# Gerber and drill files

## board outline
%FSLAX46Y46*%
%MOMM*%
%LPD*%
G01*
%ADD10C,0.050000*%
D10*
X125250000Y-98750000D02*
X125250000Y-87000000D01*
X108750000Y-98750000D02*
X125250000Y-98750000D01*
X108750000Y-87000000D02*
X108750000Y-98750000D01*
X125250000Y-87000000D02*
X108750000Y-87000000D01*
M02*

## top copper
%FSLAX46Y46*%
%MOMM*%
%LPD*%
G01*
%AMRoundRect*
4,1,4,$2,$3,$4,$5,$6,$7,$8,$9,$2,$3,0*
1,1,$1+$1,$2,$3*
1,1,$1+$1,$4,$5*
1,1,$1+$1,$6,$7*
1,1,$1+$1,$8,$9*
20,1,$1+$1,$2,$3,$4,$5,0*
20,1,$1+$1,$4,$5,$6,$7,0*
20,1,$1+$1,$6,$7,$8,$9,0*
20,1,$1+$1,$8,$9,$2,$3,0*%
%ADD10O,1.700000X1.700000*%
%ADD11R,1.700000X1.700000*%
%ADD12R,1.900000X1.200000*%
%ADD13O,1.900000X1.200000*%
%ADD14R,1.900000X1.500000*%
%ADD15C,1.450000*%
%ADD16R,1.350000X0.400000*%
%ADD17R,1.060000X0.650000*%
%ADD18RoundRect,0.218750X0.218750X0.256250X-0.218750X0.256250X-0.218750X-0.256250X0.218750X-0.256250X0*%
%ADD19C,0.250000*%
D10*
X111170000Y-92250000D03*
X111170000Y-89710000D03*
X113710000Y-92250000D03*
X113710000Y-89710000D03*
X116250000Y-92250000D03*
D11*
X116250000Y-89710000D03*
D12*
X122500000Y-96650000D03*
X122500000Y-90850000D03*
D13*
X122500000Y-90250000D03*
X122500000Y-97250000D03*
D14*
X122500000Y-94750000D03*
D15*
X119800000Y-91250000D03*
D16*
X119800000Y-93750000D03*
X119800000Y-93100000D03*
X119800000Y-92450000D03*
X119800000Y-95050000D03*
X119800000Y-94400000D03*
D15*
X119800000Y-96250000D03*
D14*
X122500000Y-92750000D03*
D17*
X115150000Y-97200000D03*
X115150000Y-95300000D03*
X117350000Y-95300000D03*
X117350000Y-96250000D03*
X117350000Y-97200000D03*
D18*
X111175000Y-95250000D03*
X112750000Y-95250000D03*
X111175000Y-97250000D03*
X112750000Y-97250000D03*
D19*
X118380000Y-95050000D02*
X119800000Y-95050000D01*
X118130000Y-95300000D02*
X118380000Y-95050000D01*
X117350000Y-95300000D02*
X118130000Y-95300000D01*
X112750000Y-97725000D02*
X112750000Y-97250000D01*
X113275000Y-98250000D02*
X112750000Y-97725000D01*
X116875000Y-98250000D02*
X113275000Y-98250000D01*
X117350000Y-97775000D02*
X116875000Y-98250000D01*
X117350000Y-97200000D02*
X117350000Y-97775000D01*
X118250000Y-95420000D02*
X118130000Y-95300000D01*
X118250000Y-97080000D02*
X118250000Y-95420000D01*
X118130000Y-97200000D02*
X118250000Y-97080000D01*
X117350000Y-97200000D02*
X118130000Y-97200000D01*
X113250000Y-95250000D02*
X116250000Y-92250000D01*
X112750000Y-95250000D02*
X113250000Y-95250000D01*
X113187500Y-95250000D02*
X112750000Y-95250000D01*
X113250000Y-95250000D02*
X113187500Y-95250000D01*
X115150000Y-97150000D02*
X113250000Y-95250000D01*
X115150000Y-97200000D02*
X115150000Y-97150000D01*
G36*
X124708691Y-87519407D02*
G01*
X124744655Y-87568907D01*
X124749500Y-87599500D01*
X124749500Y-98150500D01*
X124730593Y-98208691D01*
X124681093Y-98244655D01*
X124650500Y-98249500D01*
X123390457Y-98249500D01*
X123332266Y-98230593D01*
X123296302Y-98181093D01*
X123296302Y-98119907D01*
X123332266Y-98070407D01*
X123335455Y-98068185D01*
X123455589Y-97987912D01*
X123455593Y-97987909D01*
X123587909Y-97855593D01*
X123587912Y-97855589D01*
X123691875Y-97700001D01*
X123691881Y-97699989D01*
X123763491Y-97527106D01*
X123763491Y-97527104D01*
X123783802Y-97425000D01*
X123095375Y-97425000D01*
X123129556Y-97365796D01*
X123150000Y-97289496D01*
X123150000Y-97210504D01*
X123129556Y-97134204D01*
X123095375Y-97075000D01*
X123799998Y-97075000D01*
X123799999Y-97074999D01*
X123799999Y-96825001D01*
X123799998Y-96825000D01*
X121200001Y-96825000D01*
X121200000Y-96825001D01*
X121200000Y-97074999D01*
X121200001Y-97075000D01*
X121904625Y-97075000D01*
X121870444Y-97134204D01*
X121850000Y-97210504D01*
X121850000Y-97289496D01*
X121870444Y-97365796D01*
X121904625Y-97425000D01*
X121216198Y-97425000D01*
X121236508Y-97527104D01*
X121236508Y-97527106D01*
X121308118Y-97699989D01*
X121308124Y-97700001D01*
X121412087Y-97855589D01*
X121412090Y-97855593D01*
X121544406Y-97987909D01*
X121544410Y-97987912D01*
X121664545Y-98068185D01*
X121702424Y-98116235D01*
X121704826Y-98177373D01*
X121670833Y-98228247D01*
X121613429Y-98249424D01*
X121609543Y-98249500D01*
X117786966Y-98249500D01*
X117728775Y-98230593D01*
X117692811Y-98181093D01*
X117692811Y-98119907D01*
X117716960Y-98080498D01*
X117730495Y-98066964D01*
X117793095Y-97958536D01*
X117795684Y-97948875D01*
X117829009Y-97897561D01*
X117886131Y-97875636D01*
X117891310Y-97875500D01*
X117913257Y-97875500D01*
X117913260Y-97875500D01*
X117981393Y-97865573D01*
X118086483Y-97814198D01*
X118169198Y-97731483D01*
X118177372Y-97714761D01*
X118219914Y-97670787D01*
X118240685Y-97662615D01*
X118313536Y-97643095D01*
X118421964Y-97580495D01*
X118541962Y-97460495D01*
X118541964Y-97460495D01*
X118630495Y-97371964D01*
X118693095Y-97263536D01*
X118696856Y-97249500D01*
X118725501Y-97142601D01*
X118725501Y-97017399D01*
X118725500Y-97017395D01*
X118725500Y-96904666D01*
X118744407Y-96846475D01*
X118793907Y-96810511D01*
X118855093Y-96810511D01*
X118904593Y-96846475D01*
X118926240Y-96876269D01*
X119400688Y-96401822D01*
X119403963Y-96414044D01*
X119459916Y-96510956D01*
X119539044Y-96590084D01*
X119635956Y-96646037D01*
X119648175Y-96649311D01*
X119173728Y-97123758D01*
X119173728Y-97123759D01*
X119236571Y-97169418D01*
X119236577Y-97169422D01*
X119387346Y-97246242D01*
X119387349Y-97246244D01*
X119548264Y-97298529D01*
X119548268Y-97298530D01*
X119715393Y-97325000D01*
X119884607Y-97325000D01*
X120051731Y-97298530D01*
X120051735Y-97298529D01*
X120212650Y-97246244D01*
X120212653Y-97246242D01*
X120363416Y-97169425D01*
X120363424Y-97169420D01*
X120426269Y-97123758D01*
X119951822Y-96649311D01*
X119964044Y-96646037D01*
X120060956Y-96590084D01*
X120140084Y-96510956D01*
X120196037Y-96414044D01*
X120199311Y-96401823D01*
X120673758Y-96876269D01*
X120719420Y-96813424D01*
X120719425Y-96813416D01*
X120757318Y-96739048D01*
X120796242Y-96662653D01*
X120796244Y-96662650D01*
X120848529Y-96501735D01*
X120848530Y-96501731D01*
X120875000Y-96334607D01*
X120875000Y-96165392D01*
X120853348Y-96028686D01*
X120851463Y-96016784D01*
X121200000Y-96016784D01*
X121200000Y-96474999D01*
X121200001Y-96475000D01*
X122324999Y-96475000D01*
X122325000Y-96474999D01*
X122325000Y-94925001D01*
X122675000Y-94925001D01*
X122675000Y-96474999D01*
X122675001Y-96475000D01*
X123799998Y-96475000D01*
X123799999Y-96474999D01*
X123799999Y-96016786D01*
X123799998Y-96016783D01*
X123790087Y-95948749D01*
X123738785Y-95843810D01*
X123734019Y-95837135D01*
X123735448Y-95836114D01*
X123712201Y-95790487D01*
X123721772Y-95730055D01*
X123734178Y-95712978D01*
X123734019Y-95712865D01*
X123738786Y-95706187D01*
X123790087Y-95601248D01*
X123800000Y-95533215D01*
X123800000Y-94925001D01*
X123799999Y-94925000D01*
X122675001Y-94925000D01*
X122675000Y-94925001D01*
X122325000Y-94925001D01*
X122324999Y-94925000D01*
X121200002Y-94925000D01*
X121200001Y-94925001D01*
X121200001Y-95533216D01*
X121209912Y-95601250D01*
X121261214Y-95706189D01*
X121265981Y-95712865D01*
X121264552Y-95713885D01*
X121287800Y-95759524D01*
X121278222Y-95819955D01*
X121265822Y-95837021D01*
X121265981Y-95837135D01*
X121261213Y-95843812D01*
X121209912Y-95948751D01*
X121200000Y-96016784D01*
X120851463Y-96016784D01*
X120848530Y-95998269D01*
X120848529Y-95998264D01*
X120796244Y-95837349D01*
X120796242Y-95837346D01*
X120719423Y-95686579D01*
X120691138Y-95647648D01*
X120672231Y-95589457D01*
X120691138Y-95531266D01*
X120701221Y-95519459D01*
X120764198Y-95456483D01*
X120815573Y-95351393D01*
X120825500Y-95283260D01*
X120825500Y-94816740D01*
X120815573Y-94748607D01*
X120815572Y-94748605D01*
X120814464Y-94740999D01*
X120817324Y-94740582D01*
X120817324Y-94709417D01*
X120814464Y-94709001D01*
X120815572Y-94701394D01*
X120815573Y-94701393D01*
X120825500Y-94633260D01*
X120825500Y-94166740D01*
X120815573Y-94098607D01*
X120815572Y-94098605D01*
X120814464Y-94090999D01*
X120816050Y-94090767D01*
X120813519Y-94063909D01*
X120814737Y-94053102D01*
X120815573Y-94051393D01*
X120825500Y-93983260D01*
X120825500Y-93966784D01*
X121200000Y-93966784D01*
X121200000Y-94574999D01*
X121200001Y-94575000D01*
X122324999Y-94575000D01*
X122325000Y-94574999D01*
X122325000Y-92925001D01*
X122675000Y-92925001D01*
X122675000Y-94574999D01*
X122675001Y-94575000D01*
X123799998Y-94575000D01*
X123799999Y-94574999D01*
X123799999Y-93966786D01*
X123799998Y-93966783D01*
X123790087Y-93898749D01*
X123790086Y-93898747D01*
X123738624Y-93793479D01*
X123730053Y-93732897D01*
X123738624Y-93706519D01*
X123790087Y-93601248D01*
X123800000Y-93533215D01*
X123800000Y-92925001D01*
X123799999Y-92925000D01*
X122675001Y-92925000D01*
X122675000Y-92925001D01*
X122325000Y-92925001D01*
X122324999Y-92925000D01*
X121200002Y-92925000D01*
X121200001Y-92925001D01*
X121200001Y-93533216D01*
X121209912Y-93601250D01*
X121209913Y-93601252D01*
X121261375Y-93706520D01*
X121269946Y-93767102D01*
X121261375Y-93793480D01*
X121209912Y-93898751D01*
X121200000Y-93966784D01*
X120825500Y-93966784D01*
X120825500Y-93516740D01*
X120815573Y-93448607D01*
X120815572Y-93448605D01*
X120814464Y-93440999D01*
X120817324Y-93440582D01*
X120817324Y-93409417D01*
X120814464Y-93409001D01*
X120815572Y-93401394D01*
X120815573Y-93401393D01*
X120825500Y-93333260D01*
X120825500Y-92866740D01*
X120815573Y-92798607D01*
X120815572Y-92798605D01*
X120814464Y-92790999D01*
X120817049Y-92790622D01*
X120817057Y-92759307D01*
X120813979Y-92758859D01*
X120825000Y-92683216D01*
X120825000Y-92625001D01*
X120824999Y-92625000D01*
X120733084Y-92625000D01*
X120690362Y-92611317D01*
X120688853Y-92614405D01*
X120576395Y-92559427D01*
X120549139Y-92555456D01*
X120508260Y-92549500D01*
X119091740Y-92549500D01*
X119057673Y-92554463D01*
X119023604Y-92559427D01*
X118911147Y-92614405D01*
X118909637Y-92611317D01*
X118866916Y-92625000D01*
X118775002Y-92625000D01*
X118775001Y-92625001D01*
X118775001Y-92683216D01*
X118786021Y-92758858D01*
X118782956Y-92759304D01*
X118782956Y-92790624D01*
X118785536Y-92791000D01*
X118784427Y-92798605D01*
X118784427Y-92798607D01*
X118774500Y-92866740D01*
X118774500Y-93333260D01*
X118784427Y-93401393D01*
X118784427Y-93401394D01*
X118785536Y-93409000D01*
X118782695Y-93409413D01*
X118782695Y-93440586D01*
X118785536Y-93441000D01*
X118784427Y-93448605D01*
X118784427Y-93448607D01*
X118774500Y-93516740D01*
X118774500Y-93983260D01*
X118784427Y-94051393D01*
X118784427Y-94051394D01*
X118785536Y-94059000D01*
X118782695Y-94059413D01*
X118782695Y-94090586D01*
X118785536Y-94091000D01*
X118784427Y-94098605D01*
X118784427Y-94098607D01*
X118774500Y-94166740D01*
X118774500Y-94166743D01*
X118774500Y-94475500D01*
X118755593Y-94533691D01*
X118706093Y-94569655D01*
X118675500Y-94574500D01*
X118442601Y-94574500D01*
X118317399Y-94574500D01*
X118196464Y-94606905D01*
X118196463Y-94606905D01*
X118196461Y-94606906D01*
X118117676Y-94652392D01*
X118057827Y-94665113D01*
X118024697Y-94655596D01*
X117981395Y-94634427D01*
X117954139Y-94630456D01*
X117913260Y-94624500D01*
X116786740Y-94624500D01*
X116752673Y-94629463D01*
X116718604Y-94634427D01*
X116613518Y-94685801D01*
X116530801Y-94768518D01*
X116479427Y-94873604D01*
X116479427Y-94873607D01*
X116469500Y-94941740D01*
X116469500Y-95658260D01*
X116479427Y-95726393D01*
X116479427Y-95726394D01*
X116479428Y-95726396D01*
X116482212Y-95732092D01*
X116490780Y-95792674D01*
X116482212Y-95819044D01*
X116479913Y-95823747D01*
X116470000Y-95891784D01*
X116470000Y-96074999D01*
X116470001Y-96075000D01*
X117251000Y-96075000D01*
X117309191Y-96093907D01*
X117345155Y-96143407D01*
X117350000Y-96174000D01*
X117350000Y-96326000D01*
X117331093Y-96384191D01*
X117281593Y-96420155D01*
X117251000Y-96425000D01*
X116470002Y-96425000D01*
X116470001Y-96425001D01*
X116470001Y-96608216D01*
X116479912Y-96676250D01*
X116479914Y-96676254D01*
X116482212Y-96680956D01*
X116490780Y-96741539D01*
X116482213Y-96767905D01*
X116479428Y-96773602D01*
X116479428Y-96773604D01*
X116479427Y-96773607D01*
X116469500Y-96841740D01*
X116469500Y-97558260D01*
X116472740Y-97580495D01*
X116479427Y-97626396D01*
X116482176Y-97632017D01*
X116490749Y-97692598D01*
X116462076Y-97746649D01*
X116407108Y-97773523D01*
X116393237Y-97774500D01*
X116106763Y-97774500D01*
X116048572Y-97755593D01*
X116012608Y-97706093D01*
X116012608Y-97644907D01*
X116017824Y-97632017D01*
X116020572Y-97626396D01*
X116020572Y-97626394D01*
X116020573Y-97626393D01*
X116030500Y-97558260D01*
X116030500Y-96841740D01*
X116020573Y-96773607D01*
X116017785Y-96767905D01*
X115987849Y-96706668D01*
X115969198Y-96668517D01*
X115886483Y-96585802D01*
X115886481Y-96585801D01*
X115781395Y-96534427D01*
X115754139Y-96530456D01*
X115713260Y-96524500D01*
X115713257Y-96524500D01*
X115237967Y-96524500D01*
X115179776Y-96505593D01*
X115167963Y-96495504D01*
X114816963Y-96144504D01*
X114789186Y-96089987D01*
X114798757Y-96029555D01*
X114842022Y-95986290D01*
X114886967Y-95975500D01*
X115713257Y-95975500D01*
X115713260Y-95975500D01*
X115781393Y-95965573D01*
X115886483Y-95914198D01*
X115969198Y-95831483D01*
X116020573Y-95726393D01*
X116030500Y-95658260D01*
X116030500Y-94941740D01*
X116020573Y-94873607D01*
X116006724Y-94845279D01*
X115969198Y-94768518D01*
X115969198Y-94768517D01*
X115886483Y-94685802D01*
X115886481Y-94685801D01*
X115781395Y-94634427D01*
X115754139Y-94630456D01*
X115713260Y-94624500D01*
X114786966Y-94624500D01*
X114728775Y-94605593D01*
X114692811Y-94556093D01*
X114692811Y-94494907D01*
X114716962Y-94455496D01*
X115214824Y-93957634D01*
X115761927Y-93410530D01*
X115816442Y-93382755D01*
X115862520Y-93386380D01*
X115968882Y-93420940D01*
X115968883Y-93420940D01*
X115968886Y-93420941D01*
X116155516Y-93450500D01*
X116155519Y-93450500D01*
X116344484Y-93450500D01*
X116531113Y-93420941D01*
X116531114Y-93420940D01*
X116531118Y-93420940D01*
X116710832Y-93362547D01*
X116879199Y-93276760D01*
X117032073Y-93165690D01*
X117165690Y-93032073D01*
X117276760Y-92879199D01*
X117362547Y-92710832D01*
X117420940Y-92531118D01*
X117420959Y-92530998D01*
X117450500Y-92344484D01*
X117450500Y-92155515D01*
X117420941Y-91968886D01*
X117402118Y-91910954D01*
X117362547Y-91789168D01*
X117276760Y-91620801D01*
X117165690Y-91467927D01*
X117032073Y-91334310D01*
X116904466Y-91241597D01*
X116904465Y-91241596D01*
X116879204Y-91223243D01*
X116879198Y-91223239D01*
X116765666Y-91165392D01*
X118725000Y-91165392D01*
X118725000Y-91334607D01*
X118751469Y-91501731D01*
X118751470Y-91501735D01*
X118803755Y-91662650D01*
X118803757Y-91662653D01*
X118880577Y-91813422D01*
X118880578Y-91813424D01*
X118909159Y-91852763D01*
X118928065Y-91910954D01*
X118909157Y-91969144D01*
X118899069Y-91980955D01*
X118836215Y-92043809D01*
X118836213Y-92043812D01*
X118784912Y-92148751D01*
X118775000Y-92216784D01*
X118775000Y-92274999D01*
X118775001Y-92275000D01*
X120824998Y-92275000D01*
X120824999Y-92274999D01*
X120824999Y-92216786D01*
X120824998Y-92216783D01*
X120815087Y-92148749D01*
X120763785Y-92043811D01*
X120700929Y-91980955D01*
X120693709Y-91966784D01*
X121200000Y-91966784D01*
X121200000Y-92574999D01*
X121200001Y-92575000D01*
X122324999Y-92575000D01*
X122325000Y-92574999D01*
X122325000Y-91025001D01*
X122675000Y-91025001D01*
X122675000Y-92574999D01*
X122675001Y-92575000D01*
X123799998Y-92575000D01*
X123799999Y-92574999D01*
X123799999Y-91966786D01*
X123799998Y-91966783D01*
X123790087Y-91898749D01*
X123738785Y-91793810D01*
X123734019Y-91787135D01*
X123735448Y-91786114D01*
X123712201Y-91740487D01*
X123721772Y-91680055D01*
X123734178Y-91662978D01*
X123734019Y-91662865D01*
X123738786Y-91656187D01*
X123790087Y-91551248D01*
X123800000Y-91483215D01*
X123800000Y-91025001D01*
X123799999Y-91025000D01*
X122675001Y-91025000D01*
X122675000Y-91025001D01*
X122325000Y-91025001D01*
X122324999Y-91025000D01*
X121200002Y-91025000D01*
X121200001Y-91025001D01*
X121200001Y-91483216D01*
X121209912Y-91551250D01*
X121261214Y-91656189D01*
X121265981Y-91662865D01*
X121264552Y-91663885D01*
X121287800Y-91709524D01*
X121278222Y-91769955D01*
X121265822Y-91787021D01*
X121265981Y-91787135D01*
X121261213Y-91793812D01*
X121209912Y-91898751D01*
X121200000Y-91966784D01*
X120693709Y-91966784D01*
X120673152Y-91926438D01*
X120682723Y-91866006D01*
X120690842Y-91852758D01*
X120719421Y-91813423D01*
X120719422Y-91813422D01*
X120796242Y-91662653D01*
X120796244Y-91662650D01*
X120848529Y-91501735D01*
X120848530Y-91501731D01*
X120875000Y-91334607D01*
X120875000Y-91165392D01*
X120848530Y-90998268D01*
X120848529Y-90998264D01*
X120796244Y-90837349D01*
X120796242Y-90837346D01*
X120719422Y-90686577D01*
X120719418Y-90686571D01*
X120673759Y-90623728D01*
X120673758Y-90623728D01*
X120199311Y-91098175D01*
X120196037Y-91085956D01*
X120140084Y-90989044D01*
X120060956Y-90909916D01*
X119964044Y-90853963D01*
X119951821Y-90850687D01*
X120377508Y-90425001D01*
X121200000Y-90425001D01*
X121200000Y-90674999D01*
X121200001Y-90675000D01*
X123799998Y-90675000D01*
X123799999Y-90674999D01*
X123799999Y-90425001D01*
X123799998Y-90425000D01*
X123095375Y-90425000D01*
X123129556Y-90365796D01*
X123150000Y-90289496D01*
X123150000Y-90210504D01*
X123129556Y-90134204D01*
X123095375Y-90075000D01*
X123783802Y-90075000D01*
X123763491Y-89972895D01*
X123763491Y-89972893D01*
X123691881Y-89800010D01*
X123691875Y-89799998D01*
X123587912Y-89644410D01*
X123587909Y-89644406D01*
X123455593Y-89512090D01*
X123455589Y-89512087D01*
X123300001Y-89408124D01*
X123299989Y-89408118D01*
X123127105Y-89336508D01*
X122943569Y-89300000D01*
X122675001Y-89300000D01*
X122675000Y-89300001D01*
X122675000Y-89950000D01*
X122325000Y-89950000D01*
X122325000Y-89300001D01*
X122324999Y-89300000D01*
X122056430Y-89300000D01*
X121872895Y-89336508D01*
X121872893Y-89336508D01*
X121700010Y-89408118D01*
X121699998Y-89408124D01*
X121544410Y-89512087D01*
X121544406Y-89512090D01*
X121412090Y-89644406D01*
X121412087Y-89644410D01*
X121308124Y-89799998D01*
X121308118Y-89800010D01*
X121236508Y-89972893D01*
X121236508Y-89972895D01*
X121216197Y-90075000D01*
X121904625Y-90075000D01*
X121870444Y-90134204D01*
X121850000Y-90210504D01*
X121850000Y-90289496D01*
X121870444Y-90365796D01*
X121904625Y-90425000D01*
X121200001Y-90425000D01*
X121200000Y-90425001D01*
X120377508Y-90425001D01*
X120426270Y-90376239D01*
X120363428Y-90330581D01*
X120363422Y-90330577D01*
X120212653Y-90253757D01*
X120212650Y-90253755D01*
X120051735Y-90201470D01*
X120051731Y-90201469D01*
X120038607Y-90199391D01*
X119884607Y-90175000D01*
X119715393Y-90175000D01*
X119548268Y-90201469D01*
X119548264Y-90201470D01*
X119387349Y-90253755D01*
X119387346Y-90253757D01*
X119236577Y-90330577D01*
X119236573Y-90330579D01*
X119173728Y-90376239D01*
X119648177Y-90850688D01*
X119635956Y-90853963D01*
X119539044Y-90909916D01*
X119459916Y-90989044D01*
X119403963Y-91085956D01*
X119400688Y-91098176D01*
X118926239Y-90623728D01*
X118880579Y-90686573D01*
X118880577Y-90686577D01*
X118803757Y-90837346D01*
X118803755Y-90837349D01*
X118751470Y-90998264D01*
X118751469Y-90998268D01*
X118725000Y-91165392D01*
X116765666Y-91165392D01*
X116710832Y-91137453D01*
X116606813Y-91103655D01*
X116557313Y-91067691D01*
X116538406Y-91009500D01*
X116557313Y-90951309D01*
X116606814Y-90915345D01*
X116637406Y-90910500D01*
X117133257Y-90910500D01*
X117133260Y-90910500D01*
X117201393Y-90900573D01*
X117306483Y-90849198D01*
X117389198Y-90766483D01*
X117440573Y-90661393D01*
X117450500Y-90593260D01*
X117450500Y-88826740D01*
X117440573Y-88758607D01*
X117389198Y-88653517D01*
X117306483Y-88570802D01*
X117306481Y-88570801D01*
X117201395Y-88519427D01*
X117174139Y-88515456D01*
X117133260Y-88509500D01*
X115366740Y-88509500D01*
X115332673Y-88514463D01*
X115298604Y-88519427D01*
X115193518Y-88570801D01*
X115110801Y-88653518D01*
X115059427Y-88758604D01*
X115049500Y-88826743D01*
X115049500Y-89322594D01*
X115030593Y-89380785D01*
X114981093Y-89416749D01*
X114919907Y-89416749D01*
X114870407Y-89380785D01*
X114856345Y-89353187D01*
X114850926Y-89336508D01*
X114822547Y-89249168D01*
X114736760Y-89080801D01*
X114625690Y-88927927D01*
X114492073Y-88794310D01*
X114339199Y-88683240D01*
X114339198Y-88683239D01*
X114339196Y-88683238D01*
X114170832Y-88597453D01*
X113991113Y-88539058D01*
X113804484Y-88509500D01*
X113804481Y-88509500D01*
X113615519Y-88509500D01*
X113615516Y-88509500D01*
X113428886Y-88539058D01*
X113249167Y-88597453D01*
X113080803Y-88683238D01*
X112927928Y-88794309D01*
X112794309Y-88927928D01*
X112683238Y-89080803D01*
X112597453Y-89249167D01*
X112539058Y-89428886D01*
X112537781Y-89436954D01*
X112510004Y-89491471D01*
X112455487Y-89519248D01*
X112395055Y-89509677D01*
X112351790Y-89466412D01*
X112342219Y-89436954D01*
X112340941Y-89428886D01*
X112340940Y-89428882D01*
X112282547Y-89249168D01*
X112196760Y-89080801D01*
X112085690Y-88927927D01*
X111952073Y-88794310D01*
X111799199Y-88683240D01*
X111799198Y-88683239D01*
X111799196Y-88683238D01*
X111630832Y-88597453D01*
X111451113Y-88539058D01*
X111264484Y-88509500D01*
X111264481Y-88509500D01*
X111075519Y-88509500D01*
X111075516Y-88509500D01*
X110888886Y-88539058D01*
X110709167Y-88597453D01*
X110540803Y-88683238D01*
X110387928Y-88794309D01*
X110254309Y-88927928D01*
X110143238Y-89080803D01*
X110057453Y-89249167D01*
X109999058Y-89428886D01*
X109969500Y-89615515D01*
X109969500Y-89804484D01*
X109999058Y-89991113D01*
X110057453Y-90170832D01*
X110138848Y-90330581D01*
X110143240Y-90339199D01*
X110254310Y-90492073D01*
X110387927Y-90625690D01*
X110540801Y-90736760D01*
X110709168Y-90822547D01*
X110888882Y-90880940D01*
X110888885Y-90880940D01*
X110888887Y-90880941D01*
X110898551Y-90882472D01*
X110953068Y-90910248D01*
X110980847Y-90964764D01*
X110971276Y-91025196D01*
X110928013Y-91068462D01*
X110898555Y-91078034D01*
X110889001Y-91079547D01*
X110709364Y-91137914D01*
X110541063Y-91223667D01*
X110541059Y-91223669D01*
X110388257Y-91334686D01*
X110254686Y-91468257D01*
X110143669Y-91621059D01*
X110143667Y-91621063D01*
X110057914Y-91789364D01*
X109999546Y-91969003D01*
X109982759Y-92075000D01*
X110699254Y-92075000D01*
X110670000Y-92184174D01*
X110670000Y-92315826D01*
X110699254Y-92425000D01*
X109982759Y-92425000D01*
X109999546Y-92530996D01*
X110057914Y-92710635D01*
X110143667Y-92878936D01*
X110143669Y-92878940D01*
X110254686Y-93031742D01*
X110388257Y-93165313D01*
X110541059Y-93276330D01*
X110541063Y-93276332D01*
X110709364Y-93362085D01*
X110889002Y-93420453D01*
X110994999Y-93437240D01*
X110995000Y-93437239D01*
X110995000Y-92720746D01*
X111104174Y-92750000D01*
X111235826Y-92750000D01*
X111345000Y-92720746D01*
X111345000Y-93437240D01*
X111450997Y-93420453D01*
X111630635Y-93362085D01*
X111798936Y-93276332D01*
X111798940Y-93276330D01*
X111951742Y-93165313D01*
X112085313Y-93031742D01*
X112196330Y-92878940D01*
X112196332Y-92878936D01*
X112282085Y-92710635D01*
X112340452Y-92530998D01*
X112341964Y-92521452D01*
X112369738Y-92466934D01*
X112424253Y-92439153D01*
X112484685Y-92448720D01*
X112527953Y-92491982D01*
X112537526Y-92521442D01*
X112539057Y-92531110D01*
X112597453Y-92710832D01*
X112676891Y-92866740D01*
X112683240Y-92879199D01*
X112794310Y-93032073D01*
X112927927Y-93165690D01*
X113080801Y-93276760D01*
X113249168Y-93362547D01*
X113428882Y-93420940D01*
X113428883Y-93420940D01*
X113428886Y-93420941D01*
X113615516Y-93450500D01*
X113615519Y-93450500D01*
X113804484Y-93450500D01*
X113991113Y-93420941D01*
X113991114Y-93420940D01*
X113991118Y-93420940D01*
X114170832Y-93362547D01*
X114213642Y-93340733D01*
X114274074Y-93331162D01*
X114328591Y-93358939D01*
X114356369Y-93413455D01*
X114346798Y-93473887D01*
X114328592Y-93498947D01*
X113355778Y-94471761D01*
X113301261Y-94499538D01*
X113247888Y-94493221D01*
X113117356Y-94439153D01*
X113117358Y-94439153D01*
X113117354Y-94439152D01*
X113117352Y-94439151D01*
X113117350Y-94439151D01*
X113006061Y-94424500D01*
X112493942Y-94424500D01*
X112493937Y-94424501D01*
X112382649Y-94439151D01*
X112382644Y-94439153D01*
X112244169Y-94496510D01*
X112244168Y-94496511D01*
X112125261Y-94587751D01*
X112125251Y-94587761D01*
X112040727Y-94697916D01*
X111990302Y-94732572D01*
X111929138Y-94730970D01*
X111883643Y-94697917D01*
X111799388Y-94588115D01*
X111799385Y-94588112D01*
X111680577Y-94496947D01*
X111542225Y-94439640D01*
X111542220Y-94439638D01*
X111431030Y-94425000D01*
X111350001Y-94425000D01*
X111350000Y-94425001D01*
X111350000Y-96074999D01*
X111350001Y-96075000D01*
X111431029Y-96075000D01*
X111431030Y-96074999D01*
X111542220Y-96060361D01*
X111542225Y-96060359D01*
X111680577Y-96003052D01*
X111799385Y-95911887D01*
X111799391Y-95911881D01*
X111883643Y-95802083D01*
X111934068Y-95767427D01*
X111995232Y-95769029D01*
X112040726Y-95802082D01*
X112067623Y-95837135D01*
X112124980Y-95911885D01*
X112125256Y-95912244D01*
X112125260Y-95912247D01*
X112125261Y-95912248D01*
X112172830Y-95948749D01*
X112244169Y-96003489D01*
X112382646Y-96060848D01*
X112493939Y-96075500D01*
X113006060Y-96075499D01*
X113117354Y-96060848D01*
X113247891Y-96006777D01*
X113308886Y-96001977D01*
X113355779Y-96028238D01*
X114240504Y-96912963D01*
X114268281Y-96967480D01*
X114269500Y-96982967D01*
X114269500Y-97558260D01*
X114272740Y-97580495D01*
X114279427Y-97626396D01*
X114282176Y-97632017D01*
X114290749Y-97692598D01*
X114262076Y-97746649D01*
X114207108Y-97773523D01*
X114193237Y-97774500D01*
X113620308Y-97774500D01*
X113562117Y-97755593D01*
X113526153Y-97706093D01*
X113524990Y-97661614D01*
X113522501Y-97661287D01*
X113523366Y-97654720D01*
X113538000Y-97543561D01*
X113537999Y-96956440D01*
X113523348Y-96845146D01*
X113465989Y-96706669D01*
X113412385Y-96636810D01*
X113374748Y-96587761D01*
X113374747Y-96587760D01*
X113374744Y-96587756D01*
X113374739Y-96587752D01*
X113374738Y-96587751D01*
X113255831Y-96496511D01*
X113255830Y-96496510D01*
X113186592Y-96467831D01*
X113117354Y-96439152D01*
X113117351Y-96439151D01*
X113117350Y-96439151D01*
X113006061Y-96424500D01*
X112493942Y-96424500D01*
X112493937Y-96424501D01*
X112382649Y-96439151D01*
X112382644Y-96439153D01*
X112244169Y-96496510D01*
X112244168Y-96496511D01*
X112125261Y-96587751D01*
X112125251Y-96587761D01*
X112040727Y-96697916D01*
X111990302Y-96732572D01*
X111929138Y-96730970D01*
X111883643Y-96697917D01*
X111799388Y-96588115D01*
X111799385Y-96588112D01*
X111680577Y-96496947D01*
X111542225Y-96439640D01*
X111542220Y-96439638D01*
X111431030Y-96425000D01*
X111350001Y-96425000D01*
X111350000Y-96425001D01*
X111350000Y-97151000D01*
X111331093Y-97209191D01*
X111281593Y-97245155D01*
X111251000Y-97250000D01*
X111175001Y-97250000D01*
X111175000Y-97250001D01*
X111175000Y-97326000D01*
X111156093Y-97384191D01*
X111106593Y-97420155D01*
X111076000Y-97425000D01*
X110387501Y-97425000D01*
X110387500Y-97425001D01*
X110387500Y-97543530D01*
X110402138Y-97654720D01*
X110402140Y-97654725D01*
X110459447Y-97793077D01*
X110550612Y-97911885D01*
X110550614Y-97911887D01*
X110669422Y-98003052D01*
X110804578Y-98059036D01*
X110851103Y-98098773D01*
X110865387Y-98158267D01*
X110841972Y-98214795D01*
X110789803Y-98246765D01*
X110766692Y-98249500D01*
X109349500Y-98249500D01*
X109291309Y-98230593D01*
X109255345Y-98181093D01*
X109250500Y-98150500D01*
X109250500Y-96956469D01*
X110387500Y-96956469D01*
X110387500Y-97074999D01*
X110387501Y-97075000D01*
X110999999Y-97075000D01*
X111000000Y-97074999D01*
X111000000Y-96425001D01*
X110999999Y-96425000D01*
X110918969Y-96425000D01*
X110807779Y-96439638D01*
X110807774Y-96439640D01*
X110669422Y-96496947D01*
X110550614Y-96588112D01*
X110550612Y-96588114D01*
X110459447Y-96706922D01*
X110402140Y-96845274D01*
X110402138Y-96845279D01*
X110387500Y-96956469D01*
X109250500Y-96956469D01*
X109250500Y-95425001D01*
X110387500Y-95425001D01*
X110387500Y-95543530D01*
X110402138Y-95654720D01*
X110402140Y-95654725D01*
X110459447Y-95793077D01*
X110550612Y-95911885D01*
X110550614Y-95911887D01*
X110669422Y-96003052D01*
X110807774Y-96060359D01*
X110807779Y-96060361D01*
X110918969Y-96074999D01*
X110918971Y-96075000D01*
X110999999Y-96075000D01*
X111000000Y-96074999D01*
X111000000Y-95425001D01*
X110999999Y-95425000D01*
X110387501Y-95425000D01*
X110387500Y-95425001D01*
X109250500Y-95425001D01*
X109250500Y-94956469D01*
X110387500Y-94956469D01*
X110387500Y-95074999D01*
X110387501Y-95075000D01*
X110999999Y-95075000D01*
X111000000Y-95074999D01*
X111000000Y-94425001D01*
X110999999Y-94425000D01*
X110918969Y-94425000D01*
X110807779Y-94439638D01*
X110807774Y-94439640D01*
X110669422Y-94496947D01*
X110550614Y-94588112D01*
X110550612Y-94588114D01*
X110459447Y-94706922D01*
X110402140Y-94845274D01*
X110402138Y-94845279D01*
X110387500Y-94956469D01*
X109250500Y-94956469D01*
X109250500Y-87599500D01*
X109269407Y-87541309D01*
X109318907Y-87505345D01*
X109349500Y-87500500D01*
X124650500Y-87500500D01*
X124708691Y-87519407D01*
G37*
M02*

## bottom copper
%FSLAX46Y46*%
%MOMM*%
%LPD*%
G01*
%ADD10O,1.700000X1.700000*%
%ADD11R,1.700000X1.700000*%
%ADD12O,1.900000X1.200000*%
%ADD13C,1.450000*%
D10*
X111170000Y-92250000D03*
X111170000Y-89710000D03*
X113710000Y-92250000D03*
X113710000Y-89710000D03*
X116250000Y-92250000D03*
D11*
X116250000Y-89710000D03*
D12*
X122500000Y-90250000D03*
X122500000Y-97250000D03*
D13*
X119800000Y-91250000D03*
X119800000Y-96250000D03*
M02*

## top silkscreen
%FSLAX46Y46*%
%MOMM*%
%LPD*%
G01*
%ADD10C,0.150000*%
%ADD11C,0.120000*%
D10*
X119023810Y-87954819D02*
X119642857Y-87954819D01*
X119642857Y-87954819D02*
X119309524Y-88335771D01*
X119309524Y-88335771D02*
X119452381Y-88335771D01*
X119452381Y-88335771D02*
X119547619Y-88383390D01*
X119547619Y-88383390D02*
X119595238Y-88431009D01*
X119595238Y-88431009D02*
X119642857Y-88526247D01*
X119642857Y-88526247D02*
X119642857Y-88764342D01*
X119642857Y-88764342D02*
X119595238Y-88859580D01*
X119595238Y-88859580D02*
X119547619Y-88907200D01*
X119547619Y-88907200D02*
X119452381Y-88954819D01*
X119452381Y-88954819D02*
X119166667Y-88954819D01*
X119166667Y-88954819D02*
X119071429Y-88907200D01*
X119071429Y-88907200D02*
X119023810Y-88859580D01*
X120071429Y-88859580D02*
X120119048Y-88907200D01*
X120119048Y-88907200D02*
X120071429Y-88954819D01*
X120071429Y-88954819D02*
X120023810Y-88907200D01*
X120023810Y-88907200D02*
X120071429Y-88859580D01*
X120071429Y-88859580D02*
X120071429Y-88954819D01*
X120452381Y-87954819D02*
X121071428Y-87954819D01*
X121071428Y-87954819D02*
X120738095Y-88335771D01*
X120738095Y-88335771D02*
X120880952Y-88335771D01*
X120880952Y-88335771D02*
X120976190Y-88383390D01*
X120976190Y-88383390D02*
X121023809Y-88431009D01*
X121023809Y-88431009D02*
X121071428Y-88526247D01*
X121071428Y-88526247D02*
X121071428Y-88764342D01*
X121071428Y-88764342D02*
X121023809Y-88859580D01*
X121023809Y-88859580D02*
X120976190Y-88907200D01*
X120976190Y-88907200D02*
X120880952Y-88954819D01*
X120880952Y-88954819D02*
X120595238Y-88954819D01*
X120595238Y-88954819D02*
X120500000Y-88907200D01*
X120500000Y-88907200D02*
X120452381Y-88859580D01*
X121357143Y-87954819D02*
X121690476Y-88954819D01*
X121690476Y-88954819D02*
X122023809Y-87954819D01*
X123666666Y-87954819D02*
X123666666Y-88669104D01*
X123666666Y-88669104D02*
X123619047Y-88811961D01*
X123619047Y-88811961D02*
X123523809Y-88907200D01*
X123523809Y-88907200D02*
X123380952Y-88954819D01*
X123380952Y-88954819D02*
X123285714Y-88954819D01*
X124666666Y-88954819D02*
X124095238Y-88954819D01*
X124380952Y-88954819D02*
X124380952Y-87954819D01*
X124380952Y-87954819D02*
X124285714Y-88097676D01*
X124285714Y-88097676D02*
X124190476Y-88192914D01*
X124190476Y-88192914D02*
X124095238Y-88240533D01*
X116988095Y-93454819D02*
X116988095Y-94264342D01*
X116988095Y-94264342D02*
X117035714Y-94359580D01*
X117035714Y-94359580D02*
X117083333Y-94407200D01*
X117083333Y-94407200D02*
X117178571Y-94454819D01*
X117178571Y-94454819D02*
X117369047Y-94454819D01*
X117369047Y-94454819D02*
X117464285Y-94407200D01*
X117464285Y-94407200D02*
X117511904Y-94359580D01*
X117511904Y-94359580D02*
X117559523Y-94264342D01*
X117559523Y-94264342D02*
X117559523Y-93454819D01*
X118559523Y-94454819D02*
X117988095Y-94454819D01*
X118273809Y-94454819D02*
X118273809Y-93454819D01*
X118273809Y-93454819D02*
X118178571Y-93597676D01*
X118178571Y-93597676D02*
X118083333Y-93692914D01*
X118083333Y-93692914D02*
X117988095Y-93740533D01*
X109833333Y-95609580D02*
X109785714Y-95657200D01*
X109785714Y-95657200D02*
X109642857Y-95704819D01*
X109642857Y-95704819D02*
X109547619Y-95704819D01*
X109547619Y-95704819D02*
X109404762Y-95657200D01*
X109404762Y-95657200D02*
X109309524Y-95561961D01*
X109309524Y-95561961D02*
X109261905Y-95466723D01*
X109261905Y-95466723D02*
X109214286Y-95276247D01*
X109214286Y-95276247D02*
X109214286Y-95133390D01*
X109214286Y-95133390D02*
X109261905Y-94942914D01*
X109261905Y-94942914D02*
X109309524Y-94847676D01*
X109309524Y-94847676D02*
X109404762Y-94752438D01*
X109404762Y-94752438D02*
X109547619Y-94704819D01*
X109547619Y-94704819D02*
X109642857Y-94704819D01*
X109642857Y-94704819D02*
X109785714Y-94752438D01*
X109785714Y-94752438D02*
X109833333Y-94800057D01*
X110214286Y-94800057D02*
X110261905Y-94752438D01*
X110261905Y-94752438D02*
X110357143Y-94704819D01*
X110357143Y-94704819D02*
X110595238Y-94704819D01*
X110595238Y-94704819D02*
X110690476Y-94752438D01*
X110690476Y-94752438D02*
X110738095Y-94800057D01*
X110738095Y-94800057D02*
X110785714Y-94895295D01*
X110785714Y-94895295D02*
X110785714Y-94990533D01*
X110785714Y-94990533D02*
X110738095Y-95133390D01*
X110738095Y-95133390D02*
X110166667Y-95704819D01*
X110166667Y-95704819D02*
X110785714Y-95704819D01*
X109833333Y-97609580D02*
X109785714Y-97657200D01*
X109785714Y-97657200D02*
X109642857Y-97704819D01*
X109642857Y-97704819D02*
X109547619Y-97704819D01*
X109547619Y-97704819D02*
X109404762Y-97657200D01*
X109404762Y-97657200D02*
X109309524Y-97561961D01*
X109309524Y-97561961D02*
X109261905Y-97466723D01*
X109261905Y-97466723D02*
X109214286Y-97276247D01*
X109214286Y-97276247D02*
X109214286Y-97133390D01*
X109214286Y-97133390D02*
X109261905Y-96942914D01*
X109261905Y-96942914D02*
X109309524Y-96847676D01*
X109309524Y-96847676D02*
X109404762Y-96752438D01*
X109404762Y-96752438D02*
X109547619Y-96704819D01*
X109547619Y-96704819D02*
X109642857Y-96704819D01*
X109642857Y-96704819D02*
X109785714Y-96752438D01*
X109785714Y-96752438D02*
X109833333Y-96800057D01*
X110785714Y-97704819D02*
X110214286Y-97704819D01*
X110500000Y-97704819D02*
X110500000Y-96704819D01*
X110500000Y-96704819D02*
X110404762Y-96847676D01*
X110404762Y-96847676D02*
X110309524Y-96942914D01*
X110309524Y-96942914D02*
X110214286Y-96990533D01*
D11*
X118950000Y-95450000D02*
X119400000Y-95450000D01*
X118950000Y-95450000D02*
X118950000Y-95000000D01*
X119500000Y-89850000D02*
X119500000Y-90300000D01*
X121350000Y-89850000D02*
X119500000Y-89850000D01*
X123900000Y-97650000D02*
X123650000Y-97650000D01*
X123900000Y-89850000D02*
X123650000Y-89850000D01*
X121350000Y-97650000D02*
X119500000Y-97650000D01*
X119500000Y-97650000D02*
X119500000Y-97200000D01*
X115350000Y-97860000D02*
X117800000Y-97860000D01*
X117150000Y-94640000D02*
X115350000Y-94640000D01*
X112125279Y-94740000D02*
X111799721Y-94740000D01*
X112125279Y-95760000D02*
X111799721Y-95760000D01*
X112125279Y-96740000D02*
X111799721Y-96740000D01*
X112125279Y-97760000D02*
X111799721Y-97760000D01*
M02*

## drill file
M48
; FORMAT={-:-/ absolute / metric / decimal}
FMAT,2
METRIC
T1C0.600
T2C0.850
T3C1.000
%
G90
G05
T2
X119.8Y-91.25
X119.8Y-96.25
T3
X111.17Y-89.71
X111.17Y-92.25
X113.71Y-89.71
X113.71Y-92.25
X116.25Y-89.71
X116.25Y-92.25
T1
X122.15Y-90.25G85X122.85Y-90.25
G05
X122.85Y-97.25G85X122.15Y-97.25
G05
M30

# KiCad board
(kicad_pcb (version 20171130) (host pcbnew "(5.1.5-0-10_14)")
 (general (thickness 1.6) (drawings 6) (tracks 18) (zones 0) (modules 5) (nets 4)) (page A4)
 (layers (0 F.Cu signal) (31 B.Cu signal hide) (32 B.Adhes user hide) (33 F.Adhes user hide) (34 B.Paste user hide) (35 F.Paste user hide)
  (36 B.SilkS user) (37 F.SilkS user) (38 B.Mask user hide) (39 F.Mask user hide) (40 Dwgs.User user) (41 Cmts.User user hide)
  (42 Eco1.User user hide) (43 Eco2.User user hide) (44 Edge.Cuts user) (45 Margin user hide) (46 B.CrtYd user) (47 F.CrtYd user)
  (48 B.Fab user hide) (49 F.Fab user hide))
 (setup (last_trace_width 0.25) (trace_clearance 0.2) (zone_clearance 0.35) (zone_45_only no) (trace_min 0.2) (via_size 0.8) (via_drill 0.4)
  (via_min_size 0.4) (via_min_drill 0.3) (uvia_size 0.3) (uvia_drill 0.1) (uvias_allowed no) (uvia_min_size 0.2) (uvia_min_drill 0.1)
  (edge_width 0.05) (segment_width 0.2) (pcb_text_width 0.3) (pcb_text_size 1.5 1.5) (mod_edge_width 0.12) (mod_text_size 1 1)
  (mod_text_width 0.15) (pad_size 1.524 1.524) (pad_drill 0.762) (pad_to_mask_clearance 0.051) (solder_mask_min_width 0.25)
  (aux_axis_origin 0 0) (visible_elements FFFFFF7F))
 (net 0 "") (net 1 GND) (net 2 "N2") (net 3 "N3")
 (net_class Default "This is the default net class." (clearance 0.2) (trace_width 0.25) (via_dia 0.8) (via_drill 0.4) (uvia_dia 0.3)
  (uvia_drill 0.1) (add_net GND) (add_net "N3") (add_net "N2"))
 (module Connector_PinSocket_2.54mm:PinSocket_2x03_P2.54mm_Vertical (layer B.Cu) (at 116.25 89.71 90)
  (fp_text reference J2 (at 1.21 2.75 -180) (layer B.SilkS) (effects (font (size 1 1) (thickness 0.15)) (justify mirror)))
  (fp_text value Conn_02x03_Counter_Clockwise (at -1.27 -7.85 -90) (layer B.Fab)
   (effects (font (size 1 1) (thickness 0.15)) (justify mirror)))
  (pad 6 thru_hole oval (at -2.54 -5.08 90) (size 1.7 1.7) (drill 1) (layers *.Cu *.Mask) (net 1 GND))
  (pad 5 thru_hole oval (at 0 -5.08 90) (size 1.7 1.7) (drill 1) (layers *.Cu *.Mask))
  (pad 4 thru_hole oval (at -2.54 -2.54 90) (size 1.7 1.7) (drill 1) (layers *.Cu *.Mask))
  (pad 3 thru_hole oval (at 0 -2.54 90) (size 1.7 1.7) (drill 1) (layers *.Cu *.Mask))
  (pad 2 thru_hole oval (at -2.54 0 90) (size 1.7 1.7) (drill 1) (layers *.Cu *.Mask) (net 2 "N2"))
  (pad 1 thru_hole rect (at 0 0 90) (size 1.7 1.7) (drill 1) (layers *.Cu *.Mask)))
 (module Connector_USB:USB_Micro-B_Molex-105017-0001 (layer F.Cu) (at 121.2625 93.75 90)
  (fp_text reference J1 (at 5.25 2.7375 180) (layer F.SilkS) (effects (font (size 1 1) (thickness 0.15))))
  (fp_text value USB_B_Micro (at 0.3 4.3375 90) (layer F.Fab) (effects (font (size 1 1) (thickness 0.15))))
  (fp_line (start -1.7 -2.3125) (end -1.7 -1.8625) (layer F.SilkS) (width 0.12))
  (fp_line (start -1.7 -2.3125) (end -1.25 -2.3125) (layer F.SilkS) (width 0.12))
  (fp_line (start 3.9 -1.7625) (end 3.45 -1.7625) (layer F.SilkS) (width 0.12))
  (fp_line (start 3.9 0.0875) (end 3.9 -1.7625) (layer F.SilkS) (width 0.12))
  (fp_line (start -3.9 2.6375) (end -3.9 2.3875) (layer F.SilkS) (width 0.12))
  (fp_line (start 3.9 2.6375) (end 3.9 2.3875) (layer F.SilkS) (width 0.12))
  (fp_line (start -3.9 0.0875) (end -3.9 -1.7625) (layer F.SilkS) (width 0.12))
  (fp_line (start -3.9 -1.7625) (end -3.45 -1.7625) (layer F.SilkS) (width 0.12))
  (pad 6 smd rect (at -2.9 1.2375 90) (size 1.2 1.9) (layers F.Cu F.Mask) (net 1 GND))
  (pad 6 smd rect (at 2.9 1.2375 90) (size 1.2 1.9) (layers F.Cu F.Mask) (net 1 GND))
  (pad 6 thru_hole oval (at 3.5 1.2375 90) (size 1.2 1.9) (drill oval 0.6 1.3) (layers *.Cu *.Mask) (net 1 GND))
  (pad 6 thru_hole oval (at -3.5 1.2375 270) (size 1.2 1.9) (drill oval 0.6 1.3) (layers *.Cu *.Mask) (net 1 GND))
  (pad 6 smd rect (at -1 1.2375 90) (size 1.5 1.9) (layers F.Cu F.Paste F.Mask) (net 1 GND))
  (pad 6 thru_hole circle (at 2.5 -1.4625 90) (size 1.45 1.45) (drill 0.85) (layers *.Cu *.Mask) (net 1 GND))
  (pad 3 smd rect (at 0 -1.4625 90) (size 0.4 1.35) (layers F.Cu F.Paste F.Mask))
  (pad 4 smd rect (at 0.65 -1.4625 90) (size 0.4 1.35) (layers F.Cu F.Paste F.Mask))
  (pad 5 smd rect (at 1.3 -1.4625 90) (size 0.4 1.35) (layers F.Cu F.Paste F.Mask) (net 1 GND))
  (pad 1 smd rect (at -1.3 -1.4625 90) (size 0.4 1.35) (layers F.Cu F.Paste F.Mask) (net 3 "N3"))
  (pad 2 smd rect (at -0.65 -1.4625 90) (size 0.4 1.35) (layers F.Cu F.Paste F.Mask))
  (pad 6 thru_hole circle (at -2.5 -1.4625 90) (size 1.45 1.45) (drill 0.85) (layers *.Cu *.Mask) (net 1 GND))
  (pad 6 smd rect (at 1 1.2375 90) (size 1.5 1.9) (layers F.Cu F.Paste F.Mask) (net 1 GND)))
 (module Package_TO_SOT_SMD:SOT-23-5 (layer F.Cu) (at 116.25 96.25 180)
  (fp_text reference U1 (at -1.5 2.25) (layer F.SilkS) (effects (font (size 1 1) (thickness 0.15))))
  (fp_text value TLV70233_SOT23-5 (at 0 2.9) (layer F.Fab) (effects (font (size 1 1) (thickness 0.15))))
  (fp_line (start 0.9 -1.61) (end -1.55 -1.61) (layer F.SilkS) (width 0.12))
  (fp_line (start -0.9 1.61) (end 0.9 1.61) (layer F.SilkS) (width 0.12))
  (pad 5 smd rect (at 1.1 -0.95 180) (size 1.06 0.65) (layers F.Cu F.Paste F.Mask) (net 2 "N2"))
  (pad 4 smd rect (at 1.1 0.95 180) (size 1.06 0.65) (layers F.Cu F.Paste F.Mask))
  (pad 3 smd rect (at -1.1 0.95 180) (size 1.06 0.65) (layers F.Cu F.Paste F.Mask) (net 3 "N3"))
  (pad 2 smd rect (at -1.1 0 180) (size 1.06 0.65) (layers F.Cu F.Paste F.Mask) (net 1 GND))
  (pad 1 smd rect (at -1.1 -0.95 180) (size 1.06 0.65) (layers F.Cu F.Paste F.Mask) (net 3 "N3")))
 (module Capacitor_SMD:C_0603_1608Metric (layer F.Cu) (at 111.9625 95.25 180)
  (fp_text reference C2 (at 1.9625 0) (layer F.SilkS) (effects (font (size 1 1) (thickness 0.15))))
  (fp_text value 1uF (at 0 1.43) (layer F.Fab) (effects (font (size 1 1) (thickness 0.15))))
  (fp_line (start -0.162779 0.51) (end 0.162779 0.51) (layer F.SilkS) (width 0.12))
  (fp_line (start -0.162779 -0.51) (end 0.162779 -0.51) (layer F.SilkS) (width 0.12))
  (pad 2 smd roundrect (at 0.7875 0 180) (size 0.875 0.95) (layers F.Cu F.Paste F.Mask) (roundrect_rratio 0.25) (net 1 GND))
  (pad 1 smd roundrect (at -0.7875 0 180) (size 0.875 0.95) (layers F.Cu F.Paste F.Mask) (roundrect_rratio 0.25) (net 2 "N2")))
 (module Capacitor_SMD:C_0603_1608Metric (layer F.Cu) (at 111.9625 97.25 180)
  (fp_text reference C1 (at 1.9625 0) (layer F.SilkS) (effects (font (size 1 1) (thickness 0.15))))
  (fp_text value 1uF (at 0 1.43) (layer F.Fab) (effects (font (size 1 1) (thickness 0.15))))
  (fp_line (start -0.162779 0.51) (end 0.162779 0.51) (layer F.SilkS) (width 0.12))
  (fp_line (start -0.162779 -0.51) (end 0.162779 -0.51) (layer F.SilkS) (width 0.12))
  (pad 2 smd roundrect (at 0.7875 0 180) (size 0.875 0.95) (layers F.Cu F.Paste F.Mask) (roundrect_rratio 0.25) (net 1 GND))
  (pad 1 smd roundrect (at -0.7875 0 180) (size 0.875 0.95) (layers F.Cu F.Paste F.Mask) (roundrect_rratio 0.25) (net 3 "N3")))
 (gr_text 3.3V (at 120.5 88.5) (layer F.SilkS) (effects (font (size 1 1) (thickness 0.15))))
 (gr_line (start 125.25 98.75) (end 125.25 87) (layer Edge.Cuts) (width 0.05))
 (gr_line (start 108.75 98.75) (end 125.25 98.75) (layer Edge.Cuts) (width 0.05))
 (gr_line (start 108.75 87) (end 108.75 98.75) (layer Edge.Cuts) (width 0.05))
 (gr_line (start 125.25 87) (end 108.75 87) (layer Edge.Cuts) (width 0.05))
 (segment (start 118.38 95.05) (end 119.8 95.05) (width 0.25) (layer F.Cu) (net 3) (status 20))
 (segment (start 118.13 95.3) (end 118.38 95.05) (width 0.25) (layer F.Cu) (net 3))
 (segment (start 117.35 95.3) (end 118.13 95.3) (width 0.25) (layer F.Cu) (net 3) (status 10))
 (segment (start 112.75 97.725) (end 112.75 97.25) (width 0.25) (layer F.Cu) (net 3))
 (segment (start 113.275 98.25) (end 112.75 97.725) (width 0.25) (layer F.Cu) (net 3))
 (segment (start 116.875 98.25) (end 113.275 98.25) (width 0.25) (layer F.Cu) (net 3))
 (segment (start 117.35 97.775) (end 116.875 98.25) (width 0.25) (layer F.Cu) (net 3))
 (segment (start 117.35 97.2) (end 117.35 97.775) (width 0.25) (layer F.Cu) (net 3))
 (segment (start 118.25 95.42) (end 118.13 95.3) (width 0.25) (layer F.Cu) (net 3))
 (segment (start 118.25 97.08) (end 118.25 95.42) (width 0.25) (layer F.Cu) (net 3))
 (segment (start 118.13 97.2) (end 118.25 97.08) (width 0.25) (layer F.Cu) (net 3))
 (segment (start 117.35 97.2) (end 118.13 97.2) (width 0.25) (layer F.Cu) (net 3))
 (segment (start 113.25 95.25) (end 116.25 92.25) (width 0.25) (layer F.Cu) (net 2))
 (segment (start 112.75 95.25) (end 113.25 95.25) (width 0.25) (layer F.Cu) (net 2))
 (segment (start 113.1875 95.25) (end 112.75 95.25) (width 0.25) (layer F.Cu) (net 2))
 (segment (start 113.25 95.25) (end 113.1875 95.25) (width 0.25) (layer F.Cu) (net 2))
 (segment (start 115.15 97.15) (end 113.25 95.25) (width 0.25) (layer F.Cu) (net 2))
 (segment (start 115.15 97.2) (end 115.15 97.15) (width 0.25) (layer F.Cu) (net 2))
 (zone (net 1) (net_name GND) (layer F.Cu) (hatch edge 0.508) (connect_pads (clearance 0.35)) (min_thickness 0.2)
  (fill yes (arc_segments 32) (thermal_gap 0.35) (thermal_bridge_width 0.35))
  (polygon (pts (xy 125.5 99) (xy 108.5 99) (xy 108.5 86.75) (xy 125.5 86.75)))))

